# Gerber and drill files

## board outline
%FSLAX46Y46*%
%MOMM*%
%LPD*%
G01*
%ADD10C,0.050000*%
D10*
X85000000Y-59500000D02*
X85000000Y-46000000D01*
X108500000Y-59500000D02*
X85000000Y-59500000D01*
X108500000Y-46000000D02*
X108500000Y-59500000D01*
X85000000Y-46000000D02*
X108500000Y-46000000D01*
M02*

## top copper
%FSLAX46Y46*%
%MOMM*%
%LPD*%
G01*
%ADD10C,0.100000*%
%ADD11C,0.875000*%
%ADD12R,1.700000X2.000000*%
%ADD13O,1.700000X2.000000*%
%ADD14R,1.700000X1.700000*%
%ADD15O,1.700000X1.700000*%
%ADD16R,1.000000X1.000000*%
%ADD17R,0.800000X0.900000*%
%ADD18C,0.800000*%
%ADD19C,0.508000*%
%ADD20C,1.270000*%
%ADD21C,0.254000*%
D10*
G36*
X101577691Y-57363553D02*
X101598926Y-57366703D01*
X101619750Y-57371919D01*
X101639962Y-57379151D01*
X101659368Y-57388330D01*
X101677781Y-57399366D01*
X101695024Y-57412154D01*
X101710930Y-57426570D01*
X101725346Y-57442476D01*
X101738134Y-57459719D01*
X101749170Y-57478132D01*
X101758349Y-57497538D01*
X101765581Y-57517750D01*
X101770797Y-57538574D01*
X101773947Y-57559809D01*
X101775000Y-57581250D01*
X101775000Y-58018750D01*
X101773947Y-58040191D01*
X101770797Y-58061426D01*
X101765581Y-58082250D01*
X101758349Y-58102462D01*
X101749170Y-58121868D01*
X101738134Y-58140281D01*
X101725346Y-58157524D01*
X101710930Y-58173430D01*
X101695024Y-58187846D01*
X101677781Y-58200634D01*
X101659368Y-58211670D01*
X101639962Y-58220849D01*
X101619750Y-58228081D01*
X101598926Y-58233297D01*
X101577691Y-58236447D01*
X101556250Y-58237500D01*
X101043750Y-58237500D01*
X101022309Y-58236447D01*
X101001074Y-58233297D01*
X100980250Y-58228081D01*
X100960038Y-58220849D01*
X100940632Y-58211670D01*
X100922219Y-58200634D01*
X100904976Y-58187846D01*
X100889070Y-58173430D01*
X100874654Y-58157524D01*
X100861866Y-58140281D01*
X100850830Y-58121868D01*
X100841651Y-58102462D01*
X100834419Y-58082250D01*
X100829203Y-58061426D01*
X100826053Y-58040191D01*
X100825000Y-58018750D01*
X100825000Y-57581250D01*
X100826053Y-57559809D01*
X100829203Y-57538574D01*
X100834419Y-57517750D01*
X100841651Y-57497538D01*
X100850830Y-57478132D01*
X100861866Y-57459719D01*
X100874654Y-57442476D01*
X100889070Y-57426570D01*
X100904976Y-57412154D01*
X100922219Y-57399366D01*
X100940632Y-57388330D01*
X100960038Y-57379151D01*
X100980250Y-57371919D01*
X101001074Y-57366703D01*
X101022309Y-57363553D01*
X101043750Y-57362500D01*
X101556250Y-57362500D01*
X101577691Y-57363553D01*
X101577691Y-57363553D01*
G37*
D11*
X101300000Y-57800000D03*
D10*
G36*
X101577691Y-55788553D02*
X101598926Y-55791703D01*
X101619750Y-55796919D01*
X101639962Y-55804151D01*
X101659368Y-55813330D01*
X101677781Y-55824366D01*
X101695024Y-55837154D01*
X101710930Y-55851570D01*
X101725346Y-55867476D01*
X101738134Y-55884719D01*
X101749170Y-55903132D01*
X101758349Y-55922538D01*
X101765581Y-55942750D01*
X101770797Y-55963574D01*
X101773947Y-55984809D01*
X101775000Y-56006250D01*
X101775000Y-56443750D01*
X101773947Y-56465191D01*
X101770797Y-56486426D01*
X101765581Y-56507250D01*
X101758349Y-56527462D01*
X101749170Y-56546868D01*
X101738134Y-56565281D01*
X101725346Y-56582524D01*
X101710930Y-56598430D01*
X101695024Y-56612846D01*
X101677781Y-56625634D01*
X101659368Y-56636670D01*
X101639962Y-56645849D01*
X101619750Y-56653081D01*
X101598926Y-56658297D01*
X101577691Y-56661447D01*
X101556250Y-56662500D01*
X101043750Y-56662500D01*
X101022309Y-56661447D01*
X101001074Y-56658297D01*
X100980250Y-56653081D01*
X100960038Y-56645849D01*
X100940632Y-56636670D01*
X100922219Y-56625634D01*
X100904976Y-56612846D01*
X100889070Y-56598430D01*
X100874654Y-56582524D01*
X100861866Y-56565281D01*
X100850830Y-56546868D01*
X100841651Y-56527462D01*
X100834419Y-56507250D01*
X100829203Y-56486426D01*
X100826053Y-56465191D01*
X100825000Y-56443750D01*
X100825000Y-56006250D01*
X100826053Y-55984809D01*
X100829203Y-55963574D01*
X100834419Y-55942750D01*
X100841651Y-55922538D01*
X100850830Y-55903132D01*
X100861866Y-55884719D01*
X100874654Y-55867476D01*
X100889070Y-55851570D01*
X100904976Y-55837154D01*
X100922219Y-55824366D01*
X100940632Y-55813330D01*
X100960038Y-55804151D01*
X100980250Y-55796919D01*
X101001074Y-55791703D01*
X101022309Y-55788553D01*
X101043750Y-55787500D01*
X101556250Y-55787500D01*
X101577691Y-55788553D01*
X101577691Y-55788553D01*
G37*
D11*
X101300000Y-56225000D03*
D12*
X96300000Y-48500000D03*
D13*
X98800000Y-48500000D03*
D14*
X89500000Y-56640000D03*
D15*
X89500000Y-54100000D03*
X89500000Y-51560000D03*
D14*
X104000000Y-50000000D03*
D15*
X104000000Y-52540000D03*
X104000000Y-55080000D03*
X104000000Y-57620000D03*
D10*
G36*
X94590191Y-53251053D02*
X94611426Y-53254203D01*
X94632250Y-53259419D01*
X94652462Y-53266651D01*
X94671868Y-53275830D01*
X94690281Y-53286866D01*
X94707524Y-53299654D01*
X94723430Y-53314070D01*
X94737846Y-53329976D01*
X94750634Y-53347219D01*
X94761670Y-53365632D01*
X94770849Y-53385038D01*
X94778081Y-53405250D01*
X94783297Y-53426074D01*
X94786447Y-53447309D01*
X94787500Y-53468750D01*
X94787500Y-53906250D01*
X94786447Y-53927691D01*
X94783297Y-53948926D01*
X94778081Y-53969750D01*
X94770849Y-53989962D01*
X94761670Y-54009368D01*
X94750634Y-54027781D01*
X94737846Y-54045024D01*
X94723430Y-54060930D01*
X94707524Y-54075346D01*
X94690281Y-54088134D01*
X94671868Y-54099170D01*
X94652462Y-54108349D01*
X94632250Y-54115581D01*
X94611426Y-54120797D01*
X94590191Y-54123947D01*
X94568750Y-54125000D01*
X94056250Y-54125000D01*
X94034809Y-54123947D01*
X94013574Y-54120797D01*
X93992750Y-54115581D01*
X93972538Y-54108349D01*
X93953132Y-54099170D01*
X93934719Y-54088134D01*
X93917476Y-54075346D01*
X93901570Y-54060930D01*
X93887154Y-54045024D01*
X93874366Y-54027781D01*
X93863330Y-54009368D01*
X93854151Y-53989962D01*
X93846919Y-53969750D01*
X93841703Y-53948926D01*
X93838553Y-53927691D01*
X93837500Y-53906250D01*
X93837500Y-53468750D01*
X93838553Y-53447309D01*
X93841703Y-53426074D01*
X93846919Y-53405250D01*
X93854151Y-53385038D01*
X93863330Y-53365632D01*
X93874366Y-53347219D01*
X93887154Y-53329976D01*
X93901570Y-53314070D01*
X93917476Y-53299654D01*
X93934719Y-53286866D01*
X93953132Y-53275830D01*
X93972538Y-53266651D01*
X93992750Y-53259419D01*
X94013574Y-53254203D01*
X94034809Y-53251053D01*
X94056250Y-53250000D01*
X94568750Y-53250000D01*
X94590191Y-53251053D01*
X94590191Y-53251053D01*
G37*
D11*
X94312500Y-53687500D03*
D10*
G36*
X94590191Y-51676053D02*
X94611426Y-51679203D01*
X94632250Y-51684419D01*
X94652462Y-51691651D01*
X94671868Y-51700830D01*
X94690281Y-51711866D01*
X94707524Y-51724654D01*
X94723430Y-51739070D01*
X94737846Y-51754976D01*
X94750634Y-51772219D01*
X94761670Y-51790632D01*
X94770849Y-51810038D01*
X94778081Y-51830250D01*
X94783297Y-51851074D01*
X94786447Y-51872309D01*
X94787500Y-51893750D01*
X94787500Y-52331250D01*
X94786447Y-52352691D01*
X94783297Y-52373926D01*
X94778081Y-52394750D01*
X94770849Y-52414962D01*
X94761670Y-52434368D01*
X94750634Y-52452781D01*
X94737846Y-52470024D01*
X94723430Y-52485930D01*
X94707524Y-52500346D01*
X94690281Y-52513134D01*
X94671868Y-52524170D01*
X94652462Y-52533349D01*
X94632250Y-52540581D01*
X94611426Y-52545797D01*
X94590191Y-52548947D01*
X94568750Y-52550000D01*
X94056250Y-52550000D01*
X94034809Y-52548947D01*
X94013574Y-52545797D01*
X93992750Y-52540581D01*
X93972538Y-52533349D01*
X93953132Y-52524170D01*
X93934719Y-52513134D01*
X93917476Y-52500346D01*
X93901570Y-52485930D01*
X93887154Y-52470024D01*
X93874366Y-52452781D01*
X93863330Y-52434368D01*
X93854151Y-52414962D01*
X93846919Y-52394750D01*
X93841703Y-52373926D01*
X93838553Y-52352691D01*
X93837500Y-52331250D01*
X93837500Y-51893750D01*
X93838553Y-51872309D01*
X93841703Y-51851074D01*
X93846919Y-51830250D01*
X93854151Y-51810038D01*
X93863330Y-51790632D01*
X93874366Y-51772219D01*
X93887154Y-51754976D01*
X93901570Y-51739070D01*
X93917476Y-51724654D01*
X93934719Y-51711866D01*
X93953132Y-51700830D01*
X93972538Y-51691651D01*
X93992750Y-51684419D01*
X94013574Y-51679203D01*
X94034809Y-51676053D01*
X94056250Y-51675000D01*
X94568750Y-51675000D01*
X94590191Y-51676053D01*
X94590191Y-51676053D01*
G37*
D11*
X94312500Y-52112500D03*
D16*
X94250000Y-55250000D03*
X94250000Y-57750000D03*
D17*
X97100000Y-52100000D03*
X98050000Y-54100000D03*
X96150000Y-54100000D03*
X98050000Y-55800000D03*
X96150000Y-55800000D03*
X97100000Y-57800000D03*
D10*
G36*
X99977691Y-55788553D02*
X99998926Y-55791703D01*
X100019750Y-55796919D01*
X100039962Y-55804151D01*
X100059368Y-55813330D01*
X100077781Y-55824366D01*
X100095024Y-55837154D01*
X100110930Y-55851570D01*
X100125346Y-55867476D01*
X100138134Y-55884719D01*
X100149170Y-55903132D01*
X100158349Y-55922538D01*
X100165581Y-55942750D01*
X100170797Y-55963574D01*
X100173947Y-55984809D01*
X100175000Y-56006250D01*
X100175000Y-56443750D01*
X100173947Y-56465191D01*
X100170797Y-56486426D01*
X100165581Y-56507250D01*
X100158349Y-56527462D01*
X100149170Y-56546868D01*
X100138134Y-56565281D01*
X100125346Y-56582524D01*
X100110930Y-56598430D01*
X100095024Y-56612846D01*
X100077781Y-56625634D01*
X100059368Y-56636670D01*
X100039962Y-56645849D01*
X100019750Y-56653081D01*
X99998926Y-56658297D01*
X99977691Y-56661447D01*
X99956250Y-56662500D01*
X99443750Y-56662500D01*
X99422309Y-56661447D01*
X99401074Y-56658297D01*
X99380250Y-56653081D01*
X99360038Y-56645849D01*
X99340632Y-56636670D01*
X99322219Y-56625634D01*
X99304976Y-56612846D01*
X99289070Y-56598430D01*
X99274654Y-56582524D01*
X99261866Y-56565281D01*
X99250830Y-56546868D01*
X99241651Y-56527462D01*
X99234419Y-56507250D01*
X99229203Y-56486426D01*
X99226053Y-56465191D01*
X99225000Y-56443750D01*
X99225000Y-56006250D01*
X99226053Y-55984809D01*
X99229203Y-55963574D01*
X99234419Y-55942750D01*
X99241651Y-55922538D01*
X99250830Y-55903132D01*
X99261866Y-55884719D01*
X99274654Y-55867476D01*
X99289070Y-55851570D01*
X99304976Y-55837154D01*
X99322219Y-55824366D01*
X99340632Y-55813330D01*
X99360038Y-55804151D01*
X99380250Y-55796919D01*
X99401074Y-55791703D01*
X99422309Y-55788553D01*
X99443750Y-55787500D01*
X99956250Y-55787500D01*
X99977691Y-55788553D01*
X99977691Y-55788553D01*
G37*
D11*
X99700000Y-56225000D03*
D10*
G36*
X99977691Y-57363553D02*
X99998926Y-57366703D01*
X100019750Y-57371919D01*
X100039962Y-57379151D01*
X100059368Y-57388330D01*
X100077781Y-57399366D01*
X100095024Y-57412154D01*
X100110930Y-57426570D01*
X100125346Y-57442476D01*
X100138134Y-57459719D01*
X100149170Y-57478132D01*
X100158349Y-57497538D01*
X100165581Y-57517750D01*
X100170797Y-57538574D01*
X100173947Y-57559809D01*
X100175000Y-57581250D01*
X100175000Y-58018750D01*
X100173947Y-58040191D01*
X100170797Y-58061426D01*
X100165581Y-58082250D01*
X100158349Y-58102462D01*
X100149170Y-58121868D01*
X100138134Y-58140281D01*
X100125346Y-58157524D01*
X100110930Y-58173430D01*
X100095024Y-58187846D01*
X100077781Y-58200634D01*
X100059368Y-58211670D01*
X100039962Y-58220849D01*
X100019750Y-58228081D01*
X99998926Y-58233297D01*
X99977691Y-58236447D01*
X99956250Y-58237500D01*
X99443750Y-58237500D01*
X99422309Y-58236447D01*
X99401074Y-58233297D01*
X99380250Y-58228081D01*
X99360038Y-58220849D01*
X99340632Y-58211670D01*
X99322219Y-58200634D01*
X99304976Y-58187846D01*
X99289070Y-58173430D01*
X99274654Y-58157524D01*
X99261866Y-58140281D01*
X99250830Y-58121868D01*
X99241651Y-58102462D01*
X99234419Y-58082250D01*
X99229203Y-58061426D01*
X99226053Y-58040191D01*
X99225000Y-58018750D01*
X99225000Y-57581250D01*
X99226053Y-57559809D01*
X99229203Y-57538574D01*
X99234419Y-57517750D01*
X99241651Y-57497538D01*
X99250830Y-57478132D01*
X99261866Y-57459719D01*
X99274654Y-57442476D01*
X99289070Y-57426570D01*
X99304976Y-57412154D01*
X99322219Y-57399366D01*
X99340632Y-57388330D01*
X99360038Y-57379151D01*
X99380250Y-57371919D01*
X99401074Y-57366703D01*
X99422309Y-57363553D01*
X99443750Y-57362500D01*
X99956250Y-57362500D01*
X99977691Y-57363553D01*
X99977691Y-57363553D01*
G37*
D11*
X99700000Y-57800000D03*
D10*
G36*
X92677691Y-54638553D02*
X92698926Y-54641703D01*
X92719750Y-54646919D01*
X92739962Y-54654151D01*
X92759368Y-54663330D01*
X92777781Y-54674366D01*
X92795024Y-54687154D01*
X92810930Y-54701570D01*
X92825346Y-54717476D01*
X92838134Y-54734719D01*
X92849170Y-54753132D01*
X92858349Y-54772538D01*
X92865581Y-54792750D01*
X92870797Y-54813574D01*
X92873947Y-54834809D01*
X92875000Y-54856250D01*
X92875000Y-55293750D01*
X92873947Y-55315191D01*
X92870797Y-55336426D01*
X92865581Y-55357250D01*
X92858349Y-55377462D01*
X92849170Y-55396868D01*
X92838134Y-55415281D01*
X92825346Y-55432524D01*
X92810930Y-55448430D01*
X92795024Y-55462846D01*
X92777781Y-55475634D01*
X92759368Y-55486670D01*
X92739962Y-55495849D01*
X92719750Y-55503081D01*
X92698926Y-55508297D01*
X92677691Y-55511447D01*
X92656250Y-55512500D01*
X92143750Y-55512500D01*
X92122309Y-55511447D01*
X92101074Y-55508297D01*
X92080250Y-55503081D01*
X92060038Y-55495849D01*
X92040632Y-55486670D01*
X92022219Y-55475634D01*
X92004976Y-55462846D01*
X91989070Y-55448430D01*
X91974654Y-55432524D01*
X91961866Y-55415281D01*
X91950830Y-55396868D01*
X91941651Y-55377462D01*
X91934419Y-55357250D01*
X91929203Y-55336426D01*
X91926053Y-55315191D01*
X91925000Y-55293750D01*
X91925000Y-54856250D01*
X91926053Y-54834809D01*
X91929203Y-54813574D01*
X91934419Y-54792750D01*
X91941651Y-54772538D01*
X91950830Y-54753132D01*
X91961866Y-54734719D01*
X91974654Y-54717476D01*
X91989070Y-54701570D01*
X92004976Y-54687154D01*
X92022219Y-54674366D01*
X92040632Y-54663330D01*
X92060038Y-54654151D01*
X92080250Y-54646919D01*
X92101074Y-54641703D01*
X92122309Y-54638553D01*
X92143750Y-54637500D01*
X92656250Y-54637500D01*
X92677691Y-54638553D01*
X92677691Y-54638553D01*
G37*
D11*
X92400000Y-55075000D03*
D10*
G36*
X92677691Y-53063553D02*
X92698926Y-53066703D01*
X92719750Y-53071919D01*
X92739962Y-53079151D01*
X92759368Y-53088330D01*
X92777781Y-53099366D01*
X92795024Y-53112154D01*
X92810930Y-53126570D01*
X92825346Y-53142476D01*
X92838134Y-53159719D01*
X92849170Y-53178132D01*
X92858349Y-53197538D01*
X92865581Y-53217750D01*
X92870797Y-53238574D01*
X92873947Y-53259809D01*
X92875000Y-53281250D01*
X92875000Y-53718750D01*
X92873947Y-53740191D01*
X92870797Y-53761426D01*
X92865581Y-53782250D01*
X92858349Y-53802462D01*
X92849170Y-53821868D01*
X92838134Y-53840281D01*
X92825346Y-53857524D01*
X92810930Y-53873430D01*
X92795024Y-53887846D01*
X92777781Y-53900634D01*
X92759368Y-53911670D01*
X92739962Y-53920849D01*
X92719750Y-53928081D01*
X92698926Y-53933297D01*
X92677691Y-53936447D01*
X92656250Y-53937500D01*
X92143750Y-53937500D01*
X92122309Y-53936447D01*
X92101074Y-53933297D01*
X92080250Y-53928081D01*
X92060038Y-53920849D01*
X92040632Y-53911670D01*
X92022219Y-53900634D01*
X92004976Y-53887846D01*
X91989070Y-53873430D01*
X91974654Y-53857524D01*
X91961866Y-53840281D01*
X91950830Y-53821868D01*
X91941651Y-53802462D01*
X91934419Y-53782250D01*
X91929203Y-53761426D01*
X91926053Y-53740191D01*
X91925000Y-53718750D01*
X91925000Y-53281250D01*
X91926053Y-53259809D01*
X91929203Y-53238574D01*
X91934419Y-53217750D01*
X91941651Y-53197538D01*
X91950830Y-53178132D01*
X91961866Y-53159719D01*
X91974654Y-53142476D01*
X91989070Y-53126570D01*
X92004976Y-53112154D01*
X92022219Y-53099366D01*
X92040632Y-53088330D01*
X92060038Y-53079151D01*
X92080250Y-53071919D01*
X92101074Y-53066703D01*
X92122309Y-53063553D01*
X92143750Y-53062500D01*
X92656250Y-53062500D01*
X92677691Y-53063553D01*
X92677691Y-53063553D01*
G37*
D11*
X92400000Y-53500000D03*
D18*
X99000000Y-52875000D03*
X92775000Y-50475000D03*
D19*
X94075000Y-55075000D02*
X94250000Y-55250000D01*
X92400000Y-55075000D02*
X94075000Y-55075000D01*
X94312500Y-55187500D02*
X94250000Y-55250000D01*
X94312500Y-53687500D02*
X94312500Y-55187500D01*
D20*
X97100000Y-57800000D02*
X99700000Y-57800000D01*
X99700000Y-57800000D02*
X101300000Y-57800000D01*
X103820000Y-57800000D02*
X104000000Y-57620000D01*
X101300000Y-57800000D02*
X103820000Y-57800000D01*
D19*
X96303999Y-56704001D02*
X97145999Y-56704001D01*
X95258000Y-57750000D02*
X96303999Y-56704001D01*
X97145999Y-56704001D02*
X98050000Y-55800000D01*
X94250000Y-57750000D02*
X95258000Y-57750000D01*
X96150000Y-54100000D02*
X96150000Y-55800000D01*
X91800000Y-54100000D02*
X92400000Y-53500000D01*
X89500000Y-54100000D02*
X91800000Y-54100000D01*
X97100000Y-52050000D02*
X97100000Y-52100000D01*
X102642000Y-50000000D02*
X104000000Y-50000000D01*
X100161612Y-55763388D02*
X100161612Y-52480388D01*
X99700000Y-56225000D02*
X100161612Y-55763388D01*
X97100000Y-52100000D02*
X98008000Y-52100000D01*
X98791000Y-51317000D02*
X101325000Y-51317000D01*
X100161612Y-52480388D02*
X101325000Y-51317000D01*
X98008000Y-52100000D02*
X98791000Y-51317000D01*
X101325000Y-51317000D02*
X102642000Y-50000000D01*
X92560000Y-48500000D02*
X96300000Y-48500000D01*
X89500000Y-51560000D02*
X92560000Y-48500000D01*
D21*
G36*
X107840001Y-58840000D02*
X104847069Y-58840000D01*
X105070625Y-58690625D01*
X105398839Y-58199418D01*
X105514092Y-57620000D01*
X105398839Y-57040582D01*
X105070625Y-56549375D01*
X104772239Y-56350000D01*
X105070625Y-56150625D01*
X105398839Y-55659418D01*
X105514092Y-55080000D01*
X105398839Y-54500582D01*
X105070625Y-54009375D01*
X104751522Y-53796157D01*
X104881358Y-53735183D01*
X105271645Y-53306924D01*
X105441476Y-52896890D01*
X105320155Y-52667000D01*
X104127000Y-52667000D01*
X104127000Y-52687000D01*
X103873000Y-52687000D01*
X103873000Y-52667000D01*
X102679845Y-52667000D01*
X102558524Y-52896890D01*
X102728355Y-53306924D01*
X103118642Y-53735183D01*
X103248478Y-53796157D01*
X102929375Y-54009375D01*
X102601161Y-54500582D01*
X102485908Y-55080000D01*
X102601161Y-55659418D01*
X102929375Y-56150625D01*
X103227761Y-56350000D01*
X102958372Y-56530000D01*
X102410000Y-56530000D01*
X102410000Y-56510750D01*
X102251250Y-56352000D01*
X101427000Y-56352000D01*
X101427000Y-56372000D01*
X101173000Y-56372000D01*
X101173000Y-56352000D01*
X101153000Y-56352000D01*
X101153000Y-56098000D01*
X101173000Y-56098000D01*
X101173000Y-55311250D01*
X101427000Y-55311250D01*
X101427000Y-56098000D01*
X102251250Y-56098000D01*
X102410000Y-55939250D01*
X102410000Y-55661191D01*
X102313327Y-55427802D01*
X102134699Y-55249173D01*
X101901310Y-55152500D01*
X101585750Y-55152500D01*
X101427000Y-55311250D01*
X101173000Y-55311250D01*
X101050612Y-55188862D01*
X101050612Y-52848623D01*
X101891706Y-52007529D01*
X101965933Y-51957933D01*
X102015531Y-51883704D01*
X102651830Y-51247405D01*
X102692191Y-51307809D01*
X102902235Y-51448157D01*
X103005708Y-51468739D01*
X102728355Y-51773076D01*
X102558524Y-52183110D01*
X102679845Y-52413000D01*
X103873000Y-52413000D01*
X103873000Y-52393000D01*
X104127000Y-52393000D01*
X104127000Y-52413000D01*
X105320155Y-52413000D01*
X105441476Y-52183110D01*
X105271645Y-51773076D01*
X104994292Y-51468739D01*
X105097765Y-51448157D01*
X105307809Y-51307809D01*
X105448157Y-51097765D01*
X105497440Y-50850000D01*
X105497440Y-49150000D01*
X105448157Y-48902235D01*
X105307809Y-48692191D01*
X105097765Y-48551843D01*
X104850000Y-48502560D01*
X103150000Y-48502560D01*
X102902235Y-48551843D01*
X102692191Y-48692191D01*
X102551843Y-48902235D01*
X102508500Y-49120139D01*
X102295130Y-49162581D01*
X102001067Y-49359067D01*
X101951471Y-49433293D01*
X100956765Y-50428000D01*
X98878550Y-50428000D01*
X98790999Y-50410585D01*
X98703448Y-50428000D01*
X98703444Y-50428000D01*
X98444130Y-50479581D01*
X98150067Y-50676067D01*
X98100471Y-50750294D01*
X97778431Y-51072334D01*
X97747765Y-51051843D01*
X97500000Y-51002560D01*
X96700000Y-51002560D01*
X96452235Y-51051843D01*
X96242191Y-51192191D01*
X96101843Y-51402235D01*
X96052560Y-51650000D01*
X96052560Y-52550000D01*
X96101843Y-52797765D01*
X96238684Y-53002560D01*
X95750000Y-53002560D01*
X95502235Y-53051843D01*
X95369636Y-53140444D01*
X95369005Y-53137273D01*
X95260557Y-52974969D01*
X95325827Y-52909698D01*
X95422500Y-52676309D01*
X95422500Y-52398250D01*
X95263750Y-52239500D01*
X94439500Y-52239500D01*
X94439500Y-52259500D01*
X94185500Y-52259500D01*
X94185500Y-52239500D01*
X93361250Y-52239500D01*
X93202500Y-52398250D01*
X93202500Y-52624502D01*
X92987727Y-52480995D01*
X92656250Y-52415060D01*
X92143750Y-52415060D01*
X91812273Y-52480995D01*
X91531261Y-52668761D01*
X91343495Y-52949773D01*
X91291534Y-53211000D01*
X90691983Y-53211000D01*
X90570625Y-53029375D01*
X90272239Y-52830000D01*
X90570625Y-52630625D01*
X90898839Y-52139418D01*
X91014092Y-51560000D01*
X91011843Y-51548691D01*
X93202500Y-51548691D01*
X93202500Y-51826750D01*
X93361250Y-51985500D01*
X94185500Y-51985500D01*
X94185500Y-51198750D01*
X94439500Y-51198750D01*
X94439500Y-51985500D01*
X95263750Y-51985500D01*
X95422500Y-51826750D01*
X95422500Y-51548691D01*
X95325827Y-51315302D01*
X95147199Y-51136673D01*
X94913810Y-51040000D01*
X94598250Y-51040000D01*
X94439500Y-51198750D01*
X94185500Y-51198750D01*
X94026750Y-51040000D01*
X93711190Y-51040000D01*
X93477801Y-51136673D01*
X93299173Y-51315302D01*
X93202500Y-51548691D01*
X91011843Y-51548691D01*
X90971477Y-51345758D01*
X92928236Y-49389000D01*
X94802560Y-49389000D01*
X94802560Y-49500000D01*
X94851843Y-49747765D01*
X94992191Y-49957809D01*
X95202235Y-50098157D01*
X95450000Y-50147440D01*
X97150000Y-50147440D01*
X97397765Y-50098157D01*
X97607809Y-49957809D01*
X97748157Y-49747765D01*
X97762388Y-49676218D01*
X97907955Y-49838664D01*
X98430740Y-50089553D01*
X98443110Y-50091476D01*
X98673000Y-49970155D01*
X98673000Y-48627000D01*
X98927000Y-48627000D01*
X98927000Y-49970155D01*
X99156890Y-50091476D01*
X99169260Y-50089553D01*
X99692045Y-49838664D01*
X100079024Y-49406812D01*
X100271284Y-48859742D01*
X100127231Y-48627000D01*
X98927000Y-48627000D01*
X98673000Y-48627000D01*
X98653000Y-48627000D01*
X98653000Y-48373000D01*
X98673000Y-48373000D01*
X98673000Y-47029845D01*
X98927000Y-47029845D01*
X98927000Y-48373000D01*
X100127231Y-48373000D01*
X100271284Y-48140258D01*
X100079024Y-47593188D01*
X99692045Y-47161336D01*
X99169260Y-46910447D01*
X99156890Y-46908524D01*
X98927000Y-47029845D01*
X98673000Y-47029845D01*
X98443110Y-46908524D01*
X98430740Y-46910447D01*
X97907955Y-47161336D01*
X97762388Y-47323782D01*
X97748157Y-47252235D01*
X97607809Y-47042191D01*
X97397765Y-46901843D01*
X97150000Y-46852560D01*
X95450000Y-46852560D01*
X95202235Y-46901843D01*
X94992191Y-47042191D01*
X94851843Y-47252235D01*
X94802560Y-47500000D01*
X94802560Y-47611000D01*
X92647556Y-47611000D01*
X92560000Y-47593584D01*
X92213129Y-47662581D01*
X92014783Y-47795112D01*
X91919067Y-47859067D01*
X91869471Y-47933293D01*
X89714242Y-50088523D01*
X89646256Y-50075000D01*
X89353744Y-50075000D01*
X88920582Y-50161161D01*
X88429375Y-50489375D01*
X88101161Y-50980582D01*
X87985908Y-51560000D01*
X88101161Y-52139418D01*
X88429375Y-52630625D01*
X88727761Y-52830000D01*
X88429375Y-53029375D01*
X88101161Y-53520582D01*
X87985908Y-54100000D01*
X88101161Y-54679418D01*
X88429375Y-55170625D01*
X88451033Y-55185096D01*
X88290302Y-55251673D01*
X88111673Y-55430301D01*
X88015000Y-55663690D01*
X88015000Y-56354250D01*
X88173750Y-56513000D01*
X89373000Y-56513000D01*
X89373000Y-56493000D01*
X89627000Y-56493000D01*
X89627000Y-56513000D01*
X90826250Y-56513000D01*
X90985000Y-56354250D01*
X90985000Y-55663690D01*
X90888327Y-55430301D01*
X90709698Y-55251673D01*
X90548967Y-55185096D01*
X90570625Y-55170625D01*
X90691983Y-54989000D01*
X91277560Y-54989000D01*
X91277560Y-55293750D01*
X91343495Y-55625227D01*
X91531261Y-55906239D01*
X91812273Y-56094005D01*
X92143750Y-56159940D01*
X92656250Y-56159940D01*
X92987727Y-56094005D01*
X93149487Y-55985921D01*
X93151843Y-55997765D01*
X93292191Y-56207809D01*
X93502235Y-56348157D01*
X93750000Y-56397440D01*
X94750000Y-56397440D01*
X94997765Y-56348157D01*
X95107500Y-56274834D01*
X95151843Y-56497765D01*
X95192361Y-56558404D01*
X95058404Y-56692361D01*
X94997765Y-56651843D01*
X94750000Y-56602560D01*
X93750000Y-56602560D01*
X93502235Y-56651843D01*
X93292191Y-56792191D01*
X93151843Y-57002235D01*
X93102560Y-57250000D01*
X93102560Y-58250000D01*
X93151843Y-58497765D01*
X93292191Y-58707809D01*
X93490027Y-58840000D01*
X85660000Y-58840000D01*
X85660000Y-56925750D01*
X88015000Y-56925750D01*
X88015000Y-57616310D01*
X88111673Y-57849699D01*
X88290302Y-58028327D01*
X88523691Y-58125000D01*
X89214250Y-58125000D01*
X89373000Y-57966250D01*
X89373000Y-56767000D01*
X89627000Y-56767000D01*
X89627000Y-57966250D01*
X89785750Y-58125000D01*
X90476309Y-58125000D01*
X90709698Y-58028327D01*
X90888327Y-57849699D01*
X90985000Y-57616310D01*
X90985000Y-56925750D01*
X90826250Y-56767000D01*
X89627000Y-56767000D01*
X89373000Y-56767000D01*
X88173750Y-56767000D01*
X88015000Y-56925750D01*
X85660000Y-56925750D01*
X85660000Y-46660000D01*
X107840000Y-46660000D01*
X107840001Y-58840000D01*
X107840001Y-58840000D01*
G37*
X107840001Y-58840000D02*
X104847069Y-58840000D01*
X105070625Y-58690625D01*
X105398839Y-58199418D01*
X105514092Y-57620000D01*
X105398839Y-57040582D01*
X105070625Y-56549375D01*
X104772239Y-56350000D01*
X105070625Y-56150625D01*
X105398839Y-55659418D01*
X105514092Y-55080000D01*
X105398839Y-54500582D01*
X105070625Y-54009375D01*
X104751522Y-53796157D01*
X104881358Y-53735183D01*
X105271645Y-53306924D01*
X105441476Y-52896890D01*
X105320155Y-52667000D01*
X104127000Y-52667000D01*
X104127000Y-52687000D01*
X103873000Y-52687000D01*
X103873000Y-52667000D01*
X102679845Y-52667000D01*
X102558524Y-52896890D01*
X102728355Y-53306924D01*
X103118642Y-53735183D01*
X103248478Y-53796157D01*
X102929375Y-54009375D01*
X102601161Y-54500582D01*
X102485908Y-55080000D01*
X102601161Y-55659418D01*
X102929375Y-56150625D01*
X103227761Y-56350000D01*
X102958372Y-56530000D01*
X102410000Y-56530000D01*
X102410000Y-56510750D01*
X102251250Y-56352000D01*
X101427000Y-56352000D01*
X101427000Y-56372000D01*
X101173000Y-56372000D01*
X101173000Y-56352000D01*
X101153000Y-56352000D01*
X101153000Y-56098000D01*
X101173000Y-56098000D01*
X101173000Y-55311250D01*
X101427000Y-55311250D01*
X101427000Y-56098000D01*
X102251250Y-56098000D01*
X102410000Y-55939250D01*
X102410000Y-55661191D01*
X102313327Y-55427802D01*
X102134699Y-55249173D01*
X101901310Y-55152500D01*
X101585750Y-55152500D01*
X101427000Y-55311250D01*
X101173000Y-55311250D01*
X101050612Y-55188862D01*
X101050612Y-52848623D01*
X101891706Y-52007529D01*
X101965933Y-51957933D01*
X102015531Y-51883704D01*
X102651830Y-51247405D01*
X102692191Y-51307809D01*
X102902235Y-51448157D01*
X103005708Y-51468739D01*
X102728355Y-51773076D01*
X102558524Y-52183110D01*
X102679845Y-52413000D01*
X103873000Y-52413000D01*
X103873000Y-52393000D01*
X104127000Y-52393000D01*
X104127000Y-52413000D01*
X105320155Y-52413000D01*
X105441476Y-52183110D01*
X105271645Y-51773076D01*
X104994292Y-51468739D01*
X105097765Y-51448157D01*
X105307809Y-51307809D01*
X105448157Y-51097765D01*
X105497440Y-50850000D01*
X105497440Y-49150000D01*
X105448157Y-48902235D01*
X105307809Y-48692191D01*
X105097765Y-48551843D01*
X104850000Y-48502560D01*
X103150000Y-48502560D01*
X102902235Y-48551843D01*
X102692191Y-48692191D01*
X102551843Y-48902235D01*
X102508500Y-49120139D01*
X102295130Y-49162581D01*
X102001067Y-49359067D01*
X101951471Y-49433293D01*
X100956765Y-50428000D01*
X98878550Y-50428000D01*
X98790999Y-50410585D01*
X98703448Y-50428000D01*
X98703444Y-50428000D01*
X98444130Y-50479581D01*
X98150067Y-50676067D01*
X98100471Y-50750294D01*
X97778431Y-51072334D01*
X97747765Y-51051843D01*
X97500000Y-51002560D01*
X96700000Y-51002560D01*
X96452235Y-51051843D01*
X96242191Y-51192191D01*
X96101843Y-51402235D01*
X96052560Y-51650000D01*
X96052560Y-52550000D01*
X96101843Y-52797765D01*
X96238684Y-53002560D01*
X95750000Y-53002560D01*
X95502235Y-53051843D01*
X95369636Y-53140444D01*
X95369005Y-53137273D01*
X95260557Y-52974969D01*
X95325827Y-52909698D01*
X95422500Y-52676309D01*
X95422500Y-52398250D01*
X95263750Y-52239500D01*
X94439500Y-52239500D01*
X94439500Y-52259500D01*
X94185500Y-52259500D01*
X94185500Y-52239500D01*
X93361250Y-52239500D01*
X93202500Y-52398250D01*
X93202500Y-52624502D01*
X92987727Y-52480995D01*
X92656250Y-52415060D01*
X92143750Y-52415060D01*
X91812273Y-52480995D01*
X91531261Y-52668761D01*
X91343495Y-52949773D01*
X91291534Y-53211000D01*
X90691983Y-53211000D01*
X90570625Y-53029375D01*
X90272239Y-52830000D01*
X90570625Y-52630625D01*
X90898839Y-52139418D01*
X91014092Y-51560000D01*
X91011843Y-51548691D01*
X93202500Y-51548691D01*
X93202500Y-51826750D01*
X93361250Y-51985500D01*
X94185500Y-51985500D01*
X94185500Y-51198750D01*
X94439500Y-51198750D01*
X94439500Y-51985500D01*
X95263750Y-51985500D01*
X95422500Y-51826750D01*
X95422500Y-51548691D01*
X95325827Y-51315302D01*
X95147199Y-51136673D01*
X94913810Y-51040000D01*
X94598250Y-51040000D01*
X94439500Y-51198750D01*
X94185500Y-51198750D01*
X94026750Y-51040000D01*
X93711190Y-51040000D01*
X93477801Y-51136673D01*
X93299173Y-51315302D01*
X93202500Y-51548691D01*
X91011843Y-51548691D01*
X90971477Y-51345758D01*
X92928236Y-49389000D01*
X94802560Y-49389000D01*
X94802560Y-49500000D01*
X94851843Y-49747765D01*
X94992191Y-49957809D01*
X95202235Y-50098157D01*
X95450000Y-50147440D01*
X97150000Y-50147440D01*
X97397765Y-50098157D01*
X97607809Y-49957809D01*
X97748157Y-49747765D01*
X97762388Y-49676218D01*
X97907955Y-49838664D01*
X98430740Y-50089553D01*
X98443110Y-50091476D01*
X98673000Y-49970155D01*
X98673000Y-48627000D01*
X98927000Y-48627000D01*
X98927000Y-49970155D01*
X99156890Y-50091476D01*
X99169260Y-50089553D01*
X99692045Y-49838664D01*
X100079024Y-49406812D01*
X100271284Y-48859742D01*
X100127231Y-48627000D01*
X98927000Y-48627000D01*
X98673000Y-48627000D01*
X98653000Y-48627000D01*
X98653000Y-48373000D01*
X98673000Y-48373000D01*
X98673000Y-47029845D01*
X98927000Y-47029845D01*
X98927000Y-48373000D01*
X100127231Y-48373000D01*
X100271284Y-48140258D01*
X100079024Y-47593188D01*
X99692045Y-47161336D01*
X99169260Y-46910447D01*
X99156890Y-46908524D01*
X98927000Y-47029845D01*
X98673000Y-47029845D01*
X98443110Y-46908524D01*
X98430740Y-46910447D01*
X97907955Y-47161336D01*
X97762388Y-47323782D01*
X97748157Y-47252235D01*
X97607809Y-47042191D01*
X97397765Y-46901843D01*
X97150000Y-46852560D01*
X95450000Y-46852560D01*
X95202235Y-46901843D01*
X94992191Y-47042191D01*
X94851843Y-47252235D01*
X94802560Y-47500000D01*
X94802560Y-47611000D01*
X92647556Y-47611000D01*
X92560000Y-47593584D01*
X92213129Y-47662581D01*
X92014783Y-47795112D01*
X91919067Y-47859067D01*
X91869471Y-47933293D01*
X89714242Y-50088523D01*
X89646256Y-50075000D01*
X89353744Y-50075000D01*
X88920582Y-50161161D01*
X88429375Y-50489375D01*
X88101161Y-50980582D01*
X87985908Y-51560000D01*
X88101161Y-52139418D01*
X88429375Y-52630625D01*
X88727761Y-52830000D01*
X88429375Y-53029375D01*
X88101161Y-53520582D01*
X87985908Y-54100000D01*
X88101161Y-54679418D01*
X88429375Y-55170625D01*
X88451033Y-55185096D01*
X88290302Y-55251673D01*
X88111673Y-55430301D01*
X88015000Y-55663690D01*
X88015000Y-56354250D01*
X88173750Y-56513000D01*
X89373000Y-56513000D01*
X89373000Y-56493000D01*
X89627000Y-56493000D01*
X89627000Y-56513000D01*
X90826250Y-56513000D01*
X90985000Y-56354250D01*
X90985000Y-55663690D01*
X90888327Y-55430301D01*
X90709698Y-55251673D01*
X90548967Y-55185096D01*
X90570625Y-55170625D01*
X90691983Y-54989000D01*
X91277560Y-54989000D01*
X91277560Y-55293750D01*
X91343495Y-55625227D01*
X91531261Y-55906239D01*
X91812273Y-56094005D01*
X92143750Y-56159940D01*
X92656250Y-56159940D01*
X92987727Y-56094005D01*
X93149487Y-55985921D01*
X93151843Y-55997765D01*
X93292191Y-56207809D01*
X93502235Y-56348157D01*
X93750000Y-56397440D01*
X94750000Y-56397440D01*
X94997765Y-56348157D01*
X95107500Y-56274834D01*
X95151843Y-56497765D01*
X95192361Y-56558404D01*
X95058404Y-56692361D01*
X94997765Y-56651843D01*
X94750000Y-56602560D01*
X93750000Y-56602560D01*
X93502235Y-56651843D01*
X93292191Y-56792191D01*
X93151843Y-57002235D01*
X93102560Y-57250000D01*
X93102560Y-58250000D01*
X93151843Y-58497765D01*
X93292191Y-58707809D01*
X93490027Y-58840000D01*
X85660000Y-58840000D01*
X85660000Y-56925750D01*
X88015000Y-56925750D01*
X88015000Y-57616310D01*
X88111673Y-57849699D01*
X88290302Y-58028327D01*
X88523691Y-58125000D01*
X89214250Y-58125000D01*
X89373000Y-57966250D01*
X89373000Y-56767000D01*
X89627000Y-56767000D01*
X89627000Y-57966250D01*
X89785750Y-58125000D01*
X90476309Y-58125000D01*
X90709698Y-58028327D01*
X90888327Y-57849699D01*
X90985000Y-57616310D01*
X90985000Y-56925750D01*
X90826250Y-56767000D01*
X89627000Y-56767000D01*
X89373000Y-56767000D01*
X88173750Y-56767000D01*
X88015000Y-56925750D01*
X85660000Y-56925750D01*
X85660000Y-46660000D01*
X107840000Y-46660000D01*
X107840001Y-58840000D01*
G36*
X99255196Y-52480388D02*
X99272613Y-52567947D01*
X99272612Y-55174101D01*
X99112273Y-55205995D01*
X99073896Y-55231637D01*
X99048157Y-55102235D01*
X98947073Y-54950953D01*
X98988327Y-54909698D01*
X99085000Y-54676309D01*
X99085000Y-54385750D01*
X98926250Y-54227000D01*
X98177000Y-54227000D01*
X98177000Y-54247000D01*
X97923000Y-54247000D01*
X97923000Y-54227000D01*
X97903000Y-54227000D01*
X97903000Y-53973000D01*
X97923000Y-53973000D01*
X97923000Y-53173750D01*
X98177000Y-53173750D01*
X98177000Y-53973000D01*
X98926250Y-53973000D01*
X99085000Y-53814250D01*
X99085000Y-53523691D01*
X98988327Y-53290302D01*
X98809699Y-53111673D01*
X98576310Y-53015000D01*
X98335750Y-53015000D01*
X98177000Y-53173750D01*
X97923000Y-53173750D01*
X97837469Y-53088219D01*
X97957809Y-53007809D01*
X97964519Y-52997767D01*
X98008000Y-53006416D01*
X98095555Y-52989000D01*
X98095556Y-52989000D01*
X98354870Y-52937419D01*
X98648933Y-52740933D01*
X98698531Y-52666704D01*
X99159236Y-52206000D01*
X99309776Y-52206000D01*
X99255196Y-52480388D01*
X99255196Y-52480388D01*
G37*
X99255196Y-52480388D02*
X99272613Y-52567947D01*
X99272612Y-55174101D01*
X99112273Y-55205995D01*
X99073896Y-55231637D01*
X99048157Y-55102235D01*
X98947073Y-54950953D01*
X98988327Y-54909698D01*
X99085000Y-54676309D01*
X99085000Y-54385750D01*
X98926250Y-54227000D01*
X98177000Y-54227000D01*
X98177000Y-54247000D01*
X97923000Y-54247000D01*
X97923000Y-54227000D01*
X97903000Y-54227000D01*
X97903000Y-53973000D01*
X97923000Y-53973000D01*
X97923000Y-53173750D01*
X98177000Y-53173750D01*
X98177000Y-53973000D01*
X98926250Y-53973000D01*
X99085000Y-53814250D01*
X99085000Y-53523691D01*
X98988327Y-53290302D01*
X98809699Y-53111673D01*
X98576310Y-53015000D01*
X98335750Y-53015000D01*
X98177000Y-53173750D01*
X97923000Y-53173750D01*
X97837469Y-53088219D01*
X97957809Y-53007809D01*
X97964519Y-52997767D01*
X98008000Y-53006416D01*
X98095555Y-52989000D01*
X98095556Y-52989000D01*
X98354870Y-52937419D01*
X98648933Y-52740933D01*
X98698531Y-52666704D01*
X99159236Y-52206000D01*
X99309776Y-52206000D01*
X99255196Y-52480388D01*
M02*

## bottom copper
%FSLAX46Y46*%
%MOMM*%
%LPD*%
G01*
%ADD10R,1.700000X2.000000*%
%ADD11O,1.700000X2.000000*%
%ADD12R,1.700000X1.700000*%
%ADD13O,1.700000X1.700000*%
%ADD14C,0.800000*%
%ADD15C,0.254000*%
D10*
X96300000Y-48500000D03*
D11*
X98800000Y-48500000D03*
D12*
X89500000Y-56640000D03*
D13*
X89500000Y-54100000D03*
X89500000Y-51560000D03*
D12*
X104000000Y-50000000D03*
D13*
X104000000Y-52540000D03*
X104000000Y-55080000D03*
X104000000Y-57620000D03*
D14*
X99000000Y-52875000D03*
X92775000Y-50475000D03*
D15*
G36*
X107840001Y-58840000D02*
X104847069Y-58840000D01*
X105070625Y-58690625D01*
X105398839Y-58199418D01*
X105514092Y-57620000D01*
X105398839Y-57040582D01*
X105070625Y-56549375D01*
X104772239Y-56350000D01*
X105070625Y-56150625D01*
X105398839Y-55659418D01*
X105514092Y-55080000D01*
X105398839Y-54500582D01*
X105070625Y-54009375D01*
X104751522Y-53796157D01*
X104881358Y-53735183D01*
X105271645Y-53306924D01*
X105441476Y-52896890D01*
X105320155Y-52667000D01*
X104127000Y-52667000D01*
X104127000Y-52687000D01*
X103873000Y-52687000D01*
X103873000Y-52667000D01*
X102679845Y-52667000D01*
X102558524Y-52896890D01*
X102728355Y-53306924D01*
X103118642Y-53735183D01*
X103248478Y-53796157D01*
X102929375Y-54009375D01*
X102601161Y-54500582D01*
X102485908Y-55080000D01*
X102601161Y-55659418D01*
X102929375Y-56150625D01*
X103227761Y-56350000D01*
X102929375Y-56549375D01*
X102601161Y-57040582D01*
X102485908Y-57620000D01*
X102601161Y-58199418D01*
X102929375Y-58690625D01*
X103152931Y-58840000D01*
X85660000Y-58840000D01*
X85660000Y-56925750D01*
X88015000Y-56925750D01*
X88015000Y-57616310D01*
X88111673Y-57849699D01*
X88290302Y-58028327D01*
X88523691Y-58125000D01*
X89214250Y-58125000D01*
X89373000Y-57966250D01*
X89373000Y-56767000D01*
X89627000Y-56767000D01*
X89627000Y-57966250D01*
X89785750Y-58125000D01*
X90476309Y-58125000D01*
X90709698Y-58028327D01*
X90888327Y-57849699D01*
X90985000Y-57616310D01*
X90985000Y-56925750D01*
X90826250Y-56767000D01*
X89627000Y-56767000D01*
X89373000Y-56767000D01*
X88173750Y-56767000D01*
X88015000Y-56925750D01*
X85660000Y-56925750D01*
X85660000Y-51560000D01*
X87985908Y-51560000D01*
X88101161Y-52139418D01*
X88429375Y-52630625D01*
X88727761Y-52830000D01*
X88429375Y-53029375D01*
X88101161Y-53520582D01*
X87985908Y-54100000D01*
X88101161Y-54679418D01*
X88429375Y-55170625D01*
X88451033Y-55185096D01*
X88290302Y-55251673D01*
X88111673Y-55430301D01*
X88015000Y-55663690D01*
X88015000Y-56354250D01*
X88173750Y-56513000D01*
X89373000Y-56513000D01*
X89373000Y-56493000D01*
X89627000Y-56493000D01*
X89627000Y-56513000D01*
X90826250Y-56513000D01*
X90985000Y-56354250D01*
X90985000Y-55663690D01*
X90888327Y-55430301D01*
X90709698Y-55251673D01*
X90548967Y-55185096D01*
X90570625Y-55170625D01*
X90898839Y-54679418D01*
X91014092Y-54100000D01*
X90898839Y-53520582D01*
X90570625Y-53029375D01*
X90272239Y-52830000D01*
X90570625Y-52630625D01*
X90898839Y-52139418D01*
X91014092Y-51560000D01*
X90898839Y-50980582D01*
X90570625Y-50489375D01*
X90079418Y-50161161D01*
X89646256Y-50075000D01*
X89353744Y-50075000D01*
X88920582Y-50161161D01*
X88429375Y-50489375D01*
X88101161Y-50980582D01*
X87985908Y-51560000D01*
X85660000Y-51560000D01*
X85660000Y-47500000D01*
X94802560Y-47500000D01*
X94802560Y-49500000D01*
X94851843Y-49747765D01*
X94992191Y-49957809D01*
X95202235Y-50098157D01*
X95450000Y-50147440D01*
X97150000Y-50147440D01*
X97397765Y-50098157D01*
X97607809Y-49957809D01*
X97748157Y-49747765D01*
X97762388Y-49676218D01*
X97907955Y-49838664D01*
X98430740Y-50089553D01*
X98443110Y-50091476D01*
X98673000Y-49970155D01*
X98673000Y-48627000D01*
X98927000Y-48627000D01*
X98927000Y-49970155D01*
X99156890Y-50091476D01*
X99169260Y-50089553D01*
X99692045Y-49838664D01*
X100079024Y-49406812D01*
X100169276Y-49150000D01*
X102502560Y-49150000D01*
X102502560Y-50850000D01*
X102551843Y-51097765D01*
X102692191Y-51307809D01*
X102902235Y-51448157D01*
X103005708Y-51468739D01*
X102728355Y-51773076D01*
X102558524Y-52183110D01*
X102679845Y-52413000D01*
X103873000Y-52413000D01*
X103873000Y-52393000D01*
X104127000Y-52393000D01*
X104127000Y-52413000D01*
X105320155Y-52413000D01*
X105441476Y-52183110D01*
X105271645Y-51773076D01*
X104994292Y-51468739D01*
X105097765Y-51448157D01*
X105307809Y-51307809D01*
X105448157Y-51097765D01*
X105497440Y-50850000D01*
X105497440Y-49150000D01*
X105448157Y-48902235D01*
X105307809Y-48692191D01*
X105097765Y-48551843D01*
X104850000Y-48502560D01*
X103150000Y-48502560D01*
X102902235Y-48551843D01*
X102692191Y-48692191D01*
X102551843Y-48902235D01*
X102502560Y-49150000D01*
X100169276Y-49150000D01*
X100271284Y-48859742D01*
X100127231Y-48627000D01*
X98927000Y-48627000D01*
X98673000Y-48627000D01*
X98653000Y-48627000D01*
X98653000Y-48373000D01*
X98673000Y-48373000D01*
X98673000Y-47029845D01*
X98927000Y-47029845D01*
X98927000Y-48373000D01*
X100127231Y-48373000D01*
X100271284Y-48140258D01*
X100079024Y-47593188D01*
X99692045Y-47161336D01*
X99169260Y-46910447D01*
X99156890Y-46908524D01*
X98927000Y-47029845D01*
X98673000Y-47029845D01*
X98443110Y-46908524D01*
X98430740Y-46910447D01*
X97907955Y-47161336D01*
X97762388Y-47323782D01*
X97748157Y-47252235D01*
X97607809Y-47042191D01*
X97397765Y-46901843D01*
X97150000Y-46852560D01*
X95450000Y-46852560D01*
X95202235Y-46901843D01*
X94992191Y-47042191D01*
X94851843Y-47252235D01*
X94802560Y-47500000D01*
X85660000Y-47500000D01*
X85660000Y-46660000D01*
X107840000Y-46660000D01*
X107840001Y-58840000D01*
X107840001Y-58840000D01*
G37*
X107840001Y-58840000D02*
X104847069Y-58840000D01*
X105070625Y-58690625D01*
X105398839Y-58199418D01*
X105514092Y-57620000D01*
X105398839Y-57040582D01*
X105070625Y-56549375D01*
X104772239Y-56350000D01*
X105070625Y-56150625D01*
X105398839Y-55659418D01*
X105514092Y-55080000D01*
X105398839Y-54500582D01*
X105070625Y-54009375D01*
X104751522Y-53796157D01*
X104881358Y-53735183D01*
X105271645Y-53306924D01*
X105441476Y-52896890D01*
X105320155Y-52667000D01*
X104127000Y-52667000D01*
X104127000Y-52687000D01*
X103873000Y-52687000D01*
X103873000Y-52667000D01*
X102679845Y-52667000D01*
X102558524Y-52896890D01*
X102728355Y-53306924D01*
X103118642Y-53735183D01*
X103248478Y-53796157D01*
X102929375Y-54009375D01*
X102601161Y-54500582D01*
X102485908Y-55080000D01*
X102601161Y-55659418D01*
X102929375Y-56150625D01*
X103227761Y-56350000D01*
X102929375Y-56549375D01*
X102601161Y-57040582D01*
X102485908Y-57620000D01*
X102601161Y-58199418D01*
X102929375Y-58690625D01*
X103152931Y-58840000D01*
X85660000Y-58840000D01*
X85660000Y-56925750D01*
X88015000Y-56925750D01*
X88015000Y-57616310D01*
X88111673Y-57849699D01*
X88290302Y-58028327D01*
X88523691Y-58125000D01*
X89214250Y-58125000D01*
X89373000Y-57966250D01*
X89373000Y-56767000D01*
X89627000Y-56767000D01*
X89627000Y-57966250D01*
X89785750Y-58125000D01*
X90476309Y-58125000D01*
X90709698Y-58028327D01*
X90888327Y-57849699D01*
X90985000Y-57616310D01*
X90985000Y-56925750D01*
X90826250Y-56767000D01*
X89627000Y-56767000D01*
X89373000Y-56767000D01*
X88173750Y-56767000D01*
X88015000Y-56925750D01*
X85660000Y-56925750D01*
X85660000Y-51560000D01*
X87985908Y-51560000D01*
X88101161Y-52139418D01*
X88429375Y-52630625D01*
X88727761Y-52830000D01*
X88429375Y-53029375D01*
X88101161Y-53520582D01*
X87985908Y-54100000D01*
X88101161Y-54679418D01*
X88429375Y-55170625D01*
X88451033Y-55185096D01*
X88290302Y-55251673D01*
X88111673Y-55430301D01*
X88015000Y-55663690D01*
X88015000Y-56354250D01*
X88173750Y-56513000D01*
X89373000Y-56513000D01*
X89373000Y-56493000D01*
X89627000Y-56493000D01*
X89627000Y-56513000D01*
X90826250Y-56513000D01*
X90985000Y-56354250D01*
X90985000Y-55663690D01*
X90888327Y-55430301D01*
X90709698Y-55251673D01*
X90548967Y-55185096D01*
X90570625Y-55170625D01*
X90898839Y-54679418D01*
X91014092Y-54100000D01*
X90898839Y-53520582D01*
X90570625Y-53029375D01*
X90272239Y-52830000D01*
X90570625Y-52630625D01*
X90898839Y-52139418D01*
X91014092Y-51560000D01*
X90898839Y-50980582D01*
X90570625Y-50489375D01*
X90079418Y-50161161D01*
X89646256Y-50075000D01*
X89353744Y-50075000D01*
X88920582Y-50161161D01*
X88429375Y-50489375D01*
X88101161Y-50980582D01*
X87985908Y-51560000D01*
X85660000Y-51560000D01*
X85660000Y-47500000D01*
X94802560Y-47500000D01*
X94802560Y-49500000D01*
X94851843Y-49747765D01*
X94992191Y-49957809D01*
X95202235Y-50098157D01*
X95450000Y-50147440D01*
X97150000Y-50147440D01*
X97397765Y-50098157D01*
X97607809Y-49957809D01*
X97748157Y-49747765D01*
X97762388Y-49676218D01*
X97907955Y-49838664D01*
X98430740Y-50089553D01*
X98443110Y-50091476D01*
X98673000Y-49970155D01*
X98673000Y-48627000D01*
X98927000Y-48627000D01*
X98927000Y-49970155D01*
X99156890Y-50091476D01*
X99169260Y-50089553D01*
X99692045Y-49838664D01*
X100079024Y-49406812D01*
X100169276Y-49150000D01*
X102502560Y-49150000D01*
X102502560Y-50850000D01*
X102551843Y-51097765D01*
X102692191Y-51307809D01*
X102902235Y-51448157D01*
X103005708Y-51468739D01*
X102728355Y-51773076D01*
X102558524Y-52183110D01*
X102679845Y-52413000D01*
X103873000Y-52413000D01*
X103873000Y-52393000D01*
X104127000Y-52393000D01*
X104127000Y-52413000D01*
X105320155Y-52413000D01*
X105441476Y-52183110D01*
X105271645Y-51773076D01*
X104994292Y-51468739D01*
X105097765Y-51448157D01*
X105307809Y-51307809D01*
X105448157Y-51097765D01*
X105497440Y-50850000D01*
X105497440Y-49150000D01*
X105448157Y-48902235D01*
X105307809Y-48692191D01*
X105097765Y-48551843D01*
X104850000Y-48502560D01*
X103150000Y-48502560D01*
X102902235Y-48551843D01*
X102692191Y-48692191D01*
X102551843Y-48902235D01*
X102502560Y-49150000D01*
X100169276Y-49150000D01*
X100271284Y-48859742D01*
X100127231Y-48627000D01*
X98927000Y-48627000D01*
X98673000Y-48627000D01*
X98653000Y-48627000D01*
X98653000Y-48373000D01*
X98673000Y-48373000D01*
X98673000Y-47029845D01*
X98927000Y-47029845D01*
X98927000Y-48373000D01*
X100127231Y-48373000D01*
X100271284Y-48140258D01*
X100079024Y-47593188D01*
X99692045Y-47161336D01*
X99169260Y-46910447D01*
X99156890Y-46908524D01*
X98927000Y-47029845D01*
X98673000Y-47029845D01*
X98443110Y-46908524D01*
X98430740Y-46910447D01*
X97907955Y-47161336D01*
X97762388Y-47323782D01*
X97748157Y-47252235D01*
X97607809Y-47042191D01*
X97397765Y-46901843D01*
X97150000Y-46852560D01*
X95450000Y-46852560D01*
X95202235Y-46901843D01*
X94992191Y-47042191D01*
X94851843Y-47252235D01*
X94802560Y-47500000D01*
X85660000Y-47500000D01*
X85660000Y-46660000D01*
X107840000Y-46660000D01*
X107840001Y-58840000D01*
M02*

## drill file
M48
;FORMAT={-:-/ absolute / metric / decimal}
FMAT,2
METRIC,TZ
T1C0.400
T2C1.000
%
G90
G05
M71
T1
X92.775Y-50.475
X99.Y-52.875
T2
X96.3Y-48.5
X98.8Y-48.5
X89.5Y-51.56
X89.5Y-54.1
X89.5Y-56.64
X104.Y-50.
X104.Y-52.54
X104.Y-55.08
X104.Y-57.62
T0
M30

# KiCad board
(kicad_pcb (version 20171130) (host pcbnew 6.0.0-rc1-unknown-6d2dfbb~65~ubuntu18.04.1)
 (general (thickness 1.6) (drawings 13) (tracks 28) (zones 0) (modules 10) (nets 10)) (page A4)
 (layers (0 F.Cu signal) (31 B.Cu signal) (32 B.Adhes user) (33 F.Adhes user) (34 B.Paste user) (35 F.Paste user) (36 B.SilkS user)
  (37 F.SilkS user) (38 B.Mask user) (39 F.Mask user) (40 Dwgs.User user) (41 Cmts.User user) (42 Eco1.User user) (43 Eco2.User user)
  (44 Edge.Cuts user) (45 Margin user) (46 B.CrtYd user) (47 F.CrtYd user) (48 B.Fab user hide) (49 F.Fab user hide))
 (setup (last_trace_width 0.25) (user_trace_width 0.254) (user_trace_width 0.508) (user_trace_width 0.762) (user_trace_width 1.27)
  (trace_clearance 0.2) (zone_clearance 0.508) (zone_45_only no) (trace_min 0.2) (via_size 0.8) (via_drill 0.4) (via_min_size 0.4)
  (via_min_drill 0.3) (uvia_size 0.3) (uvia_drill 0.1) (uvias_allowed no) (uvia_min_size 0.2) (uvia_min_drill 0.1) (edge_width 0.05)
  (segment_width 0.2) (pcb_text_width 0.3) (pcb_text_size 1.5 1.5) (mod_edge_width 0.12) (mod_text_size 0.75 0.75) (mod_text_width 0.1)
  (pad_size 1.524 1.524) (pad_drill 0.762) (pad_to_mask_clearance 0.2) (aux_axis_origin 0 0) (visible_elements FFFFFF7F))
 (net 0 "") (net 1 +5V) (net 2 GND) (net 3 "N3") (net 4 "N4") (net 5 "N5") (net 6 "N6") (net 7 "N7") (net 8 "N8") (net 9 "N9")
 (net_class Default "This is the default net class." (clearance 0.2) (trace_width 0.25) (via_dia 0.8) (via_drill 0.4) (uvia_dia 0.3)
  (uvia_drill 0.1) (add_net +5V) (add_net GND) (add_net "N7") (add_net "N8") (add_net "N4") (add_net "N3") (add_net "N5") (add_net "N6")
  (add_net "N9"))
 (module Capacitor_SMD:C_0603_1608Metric (layer F.Cu) (at 101.3 57.0125 90)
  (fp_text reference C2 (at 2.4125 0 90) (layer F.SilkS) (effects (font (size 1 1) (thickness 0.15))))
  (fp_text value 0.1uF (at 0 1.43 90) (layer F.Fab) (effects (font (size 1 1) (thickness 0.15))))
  (pad 1 smd roundrect (at -0.7875 0 90) (size 0.875 0.95) (layers F.Cu F.Paste F.Mask) (roundrect_rratio 0.25) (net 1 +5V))
  (pad 2 smd roundrect (at 0.7875 0 90) (size 0.875 0.95) (layers F.Cu F.Paste F.Mask) (roundrect_rratio 0.25) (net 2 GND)))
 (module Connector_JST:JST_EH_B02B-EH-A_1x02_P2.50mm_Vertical (layer F.Cu) (at 96.3 48.5)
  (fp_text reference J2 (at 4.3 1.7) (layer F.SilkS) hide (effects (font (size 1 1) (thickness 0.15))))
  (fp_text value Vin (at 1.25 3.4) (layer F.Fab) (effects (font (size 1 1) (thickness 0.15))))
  (pad 1 thru_hole rect (at 0 0) (size 1.7 2) (drill 1) (layers *.Cu *.Mask) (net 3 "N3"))
  (pad 2 thru_hole oval (at 2.5 0) (size 1.7 2) (drill 1) (layers *.Cu *.Mask) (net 2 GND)))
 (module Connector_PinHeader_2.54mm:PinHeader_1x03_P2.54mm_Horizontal (layer F.Cu) (at 89.5 56.64 180)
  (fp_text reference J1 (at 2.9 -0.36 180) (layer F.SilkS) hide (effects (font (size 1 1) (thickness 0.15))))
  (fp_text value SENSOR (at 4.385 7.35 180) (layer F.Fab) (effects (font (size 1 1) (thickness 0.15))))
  (pad 1 thru_hole rect (at 0 0 180) (size 1.7 1.7) (drill 1) (layers *.Cu *.Mask) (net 2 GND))
  (pad 2 thru_hole oval (at 0 2.54 180) (size 1.7 1.7) (drill 1) (layers *.Cu *.Mask) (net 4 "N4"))
  (pad 3 thru_hole oval (at 0 5.08 180) (size 1.7 1.7) (drill 1) (layers *.Cu *.Mask) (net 3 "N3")))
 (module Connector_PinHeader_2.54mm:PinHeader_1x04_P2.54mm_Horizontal (layer F.Cu) (at 104 50)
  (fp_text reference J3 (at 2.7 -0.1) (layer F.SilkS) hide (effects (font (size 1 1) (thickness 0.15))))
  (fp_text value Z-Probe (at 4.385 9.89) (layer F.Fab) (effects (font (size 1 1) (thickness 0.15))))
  (pad 1 thru_hole rect (at 0 0) (size 1.7 1.7) (drill 1) (layers *.Cu *.Mask) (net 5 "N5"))
  (pad 2 thru_hole oval (at 0 2.54) (size 1.7 1.7) (drill 1) (layers *.Cu *.Mask) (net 2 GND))
  (pad 3 thru_hole oval (at 0 5.08) (size 1.7 1.7) (drill 1) (layers *.Cu *.Mask) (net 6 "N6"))
  (pad 4 thru_hole oval (at 0 7.62) (size 1.7 1.7) (drill 1) (layers *.Cu *.Mask) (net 1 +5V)))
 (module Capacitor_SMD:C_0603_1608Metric (layer F.Cu) (at 94.3125 52.9 90)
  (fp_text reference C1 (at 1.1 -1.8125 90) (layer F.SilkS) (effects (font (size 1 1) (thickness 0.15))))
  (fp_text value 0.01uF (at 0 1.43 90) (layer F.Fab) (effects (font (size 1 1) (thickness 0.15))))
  (pad 1 smd roundrect (at -0.7875 0 90) (size 0.875 0.95) (layers F.Cu F.Paste F.Mask) (roundrect_rratio 0.25) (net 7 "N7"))
  (pad 2 smd roundrect (at 0.7875 0 90) (size 0.875 0.95) (layers F.Cu F.Paste F.Mask) (roundrect_rratio 0.25) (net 2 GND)))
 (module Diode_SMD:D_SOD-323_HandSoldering (layer F.Cu) (at 94.25 56.5 270)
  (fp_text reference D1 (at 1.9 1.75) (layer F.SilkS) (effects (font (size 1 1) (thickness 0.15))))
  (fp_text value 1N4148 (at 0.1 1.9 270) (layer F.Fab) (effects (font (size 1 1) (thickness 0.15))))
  (pad 1 smd rect (at -1.25 0 270) (size 1 1) (layers F.Cu F.Paste F.Mask) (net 7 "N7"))
  (pad 2 smd rect (at 1.25 0 270) (size 1 1) (layers F.Cu F.Paste F.Mask) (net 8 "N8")))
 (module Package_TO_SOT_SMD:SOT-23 (layer F.Cu) (at 97.1 53.1 90)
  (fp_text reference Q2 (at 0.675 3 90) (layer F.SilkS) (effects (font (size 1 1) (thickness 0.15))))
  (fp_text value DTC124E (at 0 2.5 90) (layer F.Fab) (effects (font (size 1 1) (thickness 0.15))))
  (pad 3 smd rect (at 1 0 90) (size 0.9 0.8) (layers F.Cu F.Paste F.Mask) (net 5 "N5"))
  (pad 2 smd rect (at -1 0.95 90) (size 0.9 0.8) (layers F.Cu F.Paste F.Mask) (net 2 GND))
  (pad 1 smd rect (at -1 -0.95 90) (size 0.9 0.8) (layers F.Cu F.Paste F.Mask) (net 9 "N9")))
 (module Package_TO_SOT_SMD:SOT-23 (layer F.Cu) (at 97.1 56.8 270)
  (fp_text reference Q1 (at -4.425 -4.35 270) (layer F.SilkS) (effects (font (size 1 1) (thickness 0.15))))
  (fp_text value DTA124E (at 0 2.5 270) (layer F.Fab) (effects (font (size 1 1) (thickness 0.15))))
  (pad 1 smd rect (at -1 -0.95 270) (size 0.9 0.8) (layers F.Cu F.Paste F.Mask) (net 8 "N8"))
  (pad 2 smd rect (at -1 0.95 270) (size 0.9 0.8) (layers F.Cu F.Paste F.Mask) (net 9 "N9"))
  (pad 3 smd rect (at 1 0 270) (size 0.9 0.8) (layers F.Cu F.Paste F.Mask) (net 1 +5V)))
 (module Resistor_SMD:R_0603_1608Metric (layer F.Cu) (at 99.7 57.0125 90)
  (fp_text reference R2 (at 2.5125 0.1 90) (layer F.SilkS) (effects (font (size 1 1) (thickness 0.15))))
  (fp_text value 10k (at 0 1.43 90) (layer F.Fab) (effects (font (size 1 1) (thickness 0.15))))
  (pad 2 smd roundrect (at 0.7875 0 90) (size 0.875 0.95) (layers F.Cu F.Paste F.Mask) (roundrect_rratio 0.25) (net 5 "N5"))
  (pad 1 smd roundrect (at -0.7875 0 90) (size 0.875 0.95) (layers F.Cu F.Paste F.Mask) (roundrect_rratio 0.25) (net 1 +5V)))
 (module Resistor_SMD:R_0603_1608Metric (layer F.Cu) (at 92.4 54.2875 90)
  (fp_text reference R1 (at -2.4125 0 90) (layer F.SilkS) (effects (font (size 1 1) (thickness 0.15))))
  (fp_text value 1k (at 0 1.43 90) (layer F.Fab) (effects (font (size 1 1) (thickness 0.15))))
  (pad 1 smd roundrect (at -0.7875 0 90) (size 0.875 0.95) (layers F.Cu F.Paste F.Mask) (roundrect_rratio 0.25) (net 7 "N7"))
  (pad 2 smd roundrect (at 0.7875 0 90) (size 0.875 0.95) (layers F.Cu F.Paste F.Mask) (roundrect_rratio 0.25) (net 4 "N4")))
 (gr_line (start 85 59.5) (end 85 46) (layer Edge.Cuts) (width 0.05))
 (gr_line (start 108.5 59.5) (end 85 59.5) (layer Edge.Cuts) (width 0.05))
 (gr_line (start 108.5 46) (end 108.5 59.5) (layer Edge.Cuts) (width 0.05))
 (gr_line (start 85 46) (end 108.5 46) (layer Edge.Cuts) (width 0.05))
 (segment (start 94.075 55.075) (end 94.25 55.25) (width 0.508) (layer F.Cu) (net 7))
 (segment (start 92.4 55.075) (end 94.075 55.075) (width 0.508) (layer F.Cu) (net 7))
 (segment (start 94.3125 55.1875) (end 94.25 55.25) (width 0.508) (layer F.Cu) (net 7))
 (segment (start 94.3125 53.6875) (end 94.3125 55.1875) (width 0.508) (layer F.Cu) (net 7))
 (segment (start 97.1 57.8) (end 99.7 57.8) (width 1.27) (layer F.Cu) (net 1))
 (segment (start 99.7 57.8) (end 101.3 57.8) (width 1.27) (layer F.Cu) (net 1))
 (segment (start 103.82 57.8) (end 104 57.62) (width 1.27) (layer F.Cu) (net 1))
 (segment (start 101.3 57.8) (end 103.82 57.8) (width 1.27) (layer F.Cu) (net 1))
 (segment (start 96.303999 56.704001) (end 97.145999 56.704001) (width 0.508) (layer F.Cu) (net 8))
 (segment (start 95.258 57.75) (end 96.303999 56.704001) (width 0.508) (layer F.Cu) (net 8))
 (segment (start 97.145999 56.704001) (end 98.05 55.8) (width 0.508) (layer F.Cu) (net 8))
 (segment (start 94.25 57.75) (end 95.258 57.75) (width 0.508) (layer F.Cu) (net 8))
 (segment (start 96.15 54.1) (end 96.15 55.8) (width 0.508) (layer F.Cu) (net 9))
 (via (at 99 52.875) (size 0.8) (drill 0.4) (layers F.Cu B.Cu) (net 2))
 (via (at 92.775 50.475) (size 0.8) (drill 0.4) (layers F.Cu B.Cu) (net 2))
 (segment (start 91.8 54.1) (end 92.4 53.5) (width 0.508) (layer F.Cu) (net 4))
 (segment (start 89.5 54.1) (end 91.8 54.1) (width 0.508) (layer F.Cu) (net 4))
 (segment (start 97.1 52.05) (end 97.1 52.1) (width 0.508) (layer F.Cu) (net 5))
 (segment (start 102.642 50) (end 104 50) (width 0.508) (layer F.Cu) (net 5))
 (segment (start 100.161612 55.763388) (end 100.161612 52.480388) (width 0.508) (layer F.Cu) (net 5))
 (segment (start 99.7 56.225) (end 100.161612 55.763388) (width 0.508) (layer F.Cu) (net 5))
 (segment (start 97.1 52.1) (end 98.008 52.1) (width 0.508) (layer F.Cu) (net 5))
 (segment (start 98.791 51.317) (end 101.325 51.317) (width 0.508) (layer F.Cu) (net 5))
 (segment (start 100.161612 52.480388) (end 101.325 51.317) (width 0.508) (layer F.Cu) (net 5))
 (segment (start 98.008 52.1) (end 98.791 51.317) (width 0.508) (layer F.Cu) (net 5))
 (segment (start 101.325 51.317) (end 102.642 50) (width 0.508) (layer F.Cu) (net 5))
 (segment (start 92.56 48.5) (end 96.3 48.5) (width 0.508) (layer F.Cu) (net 3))
 (segment (start 89.5 51.56) (end 92.56 48.5) (width 0.508) (layer F.Cu) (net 3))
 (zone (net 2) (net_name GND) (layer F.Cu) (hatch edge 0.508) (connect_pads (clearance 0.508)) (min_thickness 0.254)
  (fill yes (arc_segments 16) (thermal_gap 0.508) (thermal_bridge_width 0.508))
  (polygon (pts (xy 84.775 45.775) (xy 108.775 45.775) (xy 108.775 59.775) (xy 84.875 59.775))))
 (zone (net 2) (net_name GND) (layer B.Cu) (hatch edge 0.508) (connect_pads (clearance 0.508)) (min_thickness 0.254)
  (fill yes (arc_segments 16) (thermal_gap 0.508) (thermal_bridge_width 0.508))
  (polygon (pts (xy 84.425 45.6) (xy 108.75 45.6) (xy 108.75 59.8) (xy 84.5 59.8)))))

